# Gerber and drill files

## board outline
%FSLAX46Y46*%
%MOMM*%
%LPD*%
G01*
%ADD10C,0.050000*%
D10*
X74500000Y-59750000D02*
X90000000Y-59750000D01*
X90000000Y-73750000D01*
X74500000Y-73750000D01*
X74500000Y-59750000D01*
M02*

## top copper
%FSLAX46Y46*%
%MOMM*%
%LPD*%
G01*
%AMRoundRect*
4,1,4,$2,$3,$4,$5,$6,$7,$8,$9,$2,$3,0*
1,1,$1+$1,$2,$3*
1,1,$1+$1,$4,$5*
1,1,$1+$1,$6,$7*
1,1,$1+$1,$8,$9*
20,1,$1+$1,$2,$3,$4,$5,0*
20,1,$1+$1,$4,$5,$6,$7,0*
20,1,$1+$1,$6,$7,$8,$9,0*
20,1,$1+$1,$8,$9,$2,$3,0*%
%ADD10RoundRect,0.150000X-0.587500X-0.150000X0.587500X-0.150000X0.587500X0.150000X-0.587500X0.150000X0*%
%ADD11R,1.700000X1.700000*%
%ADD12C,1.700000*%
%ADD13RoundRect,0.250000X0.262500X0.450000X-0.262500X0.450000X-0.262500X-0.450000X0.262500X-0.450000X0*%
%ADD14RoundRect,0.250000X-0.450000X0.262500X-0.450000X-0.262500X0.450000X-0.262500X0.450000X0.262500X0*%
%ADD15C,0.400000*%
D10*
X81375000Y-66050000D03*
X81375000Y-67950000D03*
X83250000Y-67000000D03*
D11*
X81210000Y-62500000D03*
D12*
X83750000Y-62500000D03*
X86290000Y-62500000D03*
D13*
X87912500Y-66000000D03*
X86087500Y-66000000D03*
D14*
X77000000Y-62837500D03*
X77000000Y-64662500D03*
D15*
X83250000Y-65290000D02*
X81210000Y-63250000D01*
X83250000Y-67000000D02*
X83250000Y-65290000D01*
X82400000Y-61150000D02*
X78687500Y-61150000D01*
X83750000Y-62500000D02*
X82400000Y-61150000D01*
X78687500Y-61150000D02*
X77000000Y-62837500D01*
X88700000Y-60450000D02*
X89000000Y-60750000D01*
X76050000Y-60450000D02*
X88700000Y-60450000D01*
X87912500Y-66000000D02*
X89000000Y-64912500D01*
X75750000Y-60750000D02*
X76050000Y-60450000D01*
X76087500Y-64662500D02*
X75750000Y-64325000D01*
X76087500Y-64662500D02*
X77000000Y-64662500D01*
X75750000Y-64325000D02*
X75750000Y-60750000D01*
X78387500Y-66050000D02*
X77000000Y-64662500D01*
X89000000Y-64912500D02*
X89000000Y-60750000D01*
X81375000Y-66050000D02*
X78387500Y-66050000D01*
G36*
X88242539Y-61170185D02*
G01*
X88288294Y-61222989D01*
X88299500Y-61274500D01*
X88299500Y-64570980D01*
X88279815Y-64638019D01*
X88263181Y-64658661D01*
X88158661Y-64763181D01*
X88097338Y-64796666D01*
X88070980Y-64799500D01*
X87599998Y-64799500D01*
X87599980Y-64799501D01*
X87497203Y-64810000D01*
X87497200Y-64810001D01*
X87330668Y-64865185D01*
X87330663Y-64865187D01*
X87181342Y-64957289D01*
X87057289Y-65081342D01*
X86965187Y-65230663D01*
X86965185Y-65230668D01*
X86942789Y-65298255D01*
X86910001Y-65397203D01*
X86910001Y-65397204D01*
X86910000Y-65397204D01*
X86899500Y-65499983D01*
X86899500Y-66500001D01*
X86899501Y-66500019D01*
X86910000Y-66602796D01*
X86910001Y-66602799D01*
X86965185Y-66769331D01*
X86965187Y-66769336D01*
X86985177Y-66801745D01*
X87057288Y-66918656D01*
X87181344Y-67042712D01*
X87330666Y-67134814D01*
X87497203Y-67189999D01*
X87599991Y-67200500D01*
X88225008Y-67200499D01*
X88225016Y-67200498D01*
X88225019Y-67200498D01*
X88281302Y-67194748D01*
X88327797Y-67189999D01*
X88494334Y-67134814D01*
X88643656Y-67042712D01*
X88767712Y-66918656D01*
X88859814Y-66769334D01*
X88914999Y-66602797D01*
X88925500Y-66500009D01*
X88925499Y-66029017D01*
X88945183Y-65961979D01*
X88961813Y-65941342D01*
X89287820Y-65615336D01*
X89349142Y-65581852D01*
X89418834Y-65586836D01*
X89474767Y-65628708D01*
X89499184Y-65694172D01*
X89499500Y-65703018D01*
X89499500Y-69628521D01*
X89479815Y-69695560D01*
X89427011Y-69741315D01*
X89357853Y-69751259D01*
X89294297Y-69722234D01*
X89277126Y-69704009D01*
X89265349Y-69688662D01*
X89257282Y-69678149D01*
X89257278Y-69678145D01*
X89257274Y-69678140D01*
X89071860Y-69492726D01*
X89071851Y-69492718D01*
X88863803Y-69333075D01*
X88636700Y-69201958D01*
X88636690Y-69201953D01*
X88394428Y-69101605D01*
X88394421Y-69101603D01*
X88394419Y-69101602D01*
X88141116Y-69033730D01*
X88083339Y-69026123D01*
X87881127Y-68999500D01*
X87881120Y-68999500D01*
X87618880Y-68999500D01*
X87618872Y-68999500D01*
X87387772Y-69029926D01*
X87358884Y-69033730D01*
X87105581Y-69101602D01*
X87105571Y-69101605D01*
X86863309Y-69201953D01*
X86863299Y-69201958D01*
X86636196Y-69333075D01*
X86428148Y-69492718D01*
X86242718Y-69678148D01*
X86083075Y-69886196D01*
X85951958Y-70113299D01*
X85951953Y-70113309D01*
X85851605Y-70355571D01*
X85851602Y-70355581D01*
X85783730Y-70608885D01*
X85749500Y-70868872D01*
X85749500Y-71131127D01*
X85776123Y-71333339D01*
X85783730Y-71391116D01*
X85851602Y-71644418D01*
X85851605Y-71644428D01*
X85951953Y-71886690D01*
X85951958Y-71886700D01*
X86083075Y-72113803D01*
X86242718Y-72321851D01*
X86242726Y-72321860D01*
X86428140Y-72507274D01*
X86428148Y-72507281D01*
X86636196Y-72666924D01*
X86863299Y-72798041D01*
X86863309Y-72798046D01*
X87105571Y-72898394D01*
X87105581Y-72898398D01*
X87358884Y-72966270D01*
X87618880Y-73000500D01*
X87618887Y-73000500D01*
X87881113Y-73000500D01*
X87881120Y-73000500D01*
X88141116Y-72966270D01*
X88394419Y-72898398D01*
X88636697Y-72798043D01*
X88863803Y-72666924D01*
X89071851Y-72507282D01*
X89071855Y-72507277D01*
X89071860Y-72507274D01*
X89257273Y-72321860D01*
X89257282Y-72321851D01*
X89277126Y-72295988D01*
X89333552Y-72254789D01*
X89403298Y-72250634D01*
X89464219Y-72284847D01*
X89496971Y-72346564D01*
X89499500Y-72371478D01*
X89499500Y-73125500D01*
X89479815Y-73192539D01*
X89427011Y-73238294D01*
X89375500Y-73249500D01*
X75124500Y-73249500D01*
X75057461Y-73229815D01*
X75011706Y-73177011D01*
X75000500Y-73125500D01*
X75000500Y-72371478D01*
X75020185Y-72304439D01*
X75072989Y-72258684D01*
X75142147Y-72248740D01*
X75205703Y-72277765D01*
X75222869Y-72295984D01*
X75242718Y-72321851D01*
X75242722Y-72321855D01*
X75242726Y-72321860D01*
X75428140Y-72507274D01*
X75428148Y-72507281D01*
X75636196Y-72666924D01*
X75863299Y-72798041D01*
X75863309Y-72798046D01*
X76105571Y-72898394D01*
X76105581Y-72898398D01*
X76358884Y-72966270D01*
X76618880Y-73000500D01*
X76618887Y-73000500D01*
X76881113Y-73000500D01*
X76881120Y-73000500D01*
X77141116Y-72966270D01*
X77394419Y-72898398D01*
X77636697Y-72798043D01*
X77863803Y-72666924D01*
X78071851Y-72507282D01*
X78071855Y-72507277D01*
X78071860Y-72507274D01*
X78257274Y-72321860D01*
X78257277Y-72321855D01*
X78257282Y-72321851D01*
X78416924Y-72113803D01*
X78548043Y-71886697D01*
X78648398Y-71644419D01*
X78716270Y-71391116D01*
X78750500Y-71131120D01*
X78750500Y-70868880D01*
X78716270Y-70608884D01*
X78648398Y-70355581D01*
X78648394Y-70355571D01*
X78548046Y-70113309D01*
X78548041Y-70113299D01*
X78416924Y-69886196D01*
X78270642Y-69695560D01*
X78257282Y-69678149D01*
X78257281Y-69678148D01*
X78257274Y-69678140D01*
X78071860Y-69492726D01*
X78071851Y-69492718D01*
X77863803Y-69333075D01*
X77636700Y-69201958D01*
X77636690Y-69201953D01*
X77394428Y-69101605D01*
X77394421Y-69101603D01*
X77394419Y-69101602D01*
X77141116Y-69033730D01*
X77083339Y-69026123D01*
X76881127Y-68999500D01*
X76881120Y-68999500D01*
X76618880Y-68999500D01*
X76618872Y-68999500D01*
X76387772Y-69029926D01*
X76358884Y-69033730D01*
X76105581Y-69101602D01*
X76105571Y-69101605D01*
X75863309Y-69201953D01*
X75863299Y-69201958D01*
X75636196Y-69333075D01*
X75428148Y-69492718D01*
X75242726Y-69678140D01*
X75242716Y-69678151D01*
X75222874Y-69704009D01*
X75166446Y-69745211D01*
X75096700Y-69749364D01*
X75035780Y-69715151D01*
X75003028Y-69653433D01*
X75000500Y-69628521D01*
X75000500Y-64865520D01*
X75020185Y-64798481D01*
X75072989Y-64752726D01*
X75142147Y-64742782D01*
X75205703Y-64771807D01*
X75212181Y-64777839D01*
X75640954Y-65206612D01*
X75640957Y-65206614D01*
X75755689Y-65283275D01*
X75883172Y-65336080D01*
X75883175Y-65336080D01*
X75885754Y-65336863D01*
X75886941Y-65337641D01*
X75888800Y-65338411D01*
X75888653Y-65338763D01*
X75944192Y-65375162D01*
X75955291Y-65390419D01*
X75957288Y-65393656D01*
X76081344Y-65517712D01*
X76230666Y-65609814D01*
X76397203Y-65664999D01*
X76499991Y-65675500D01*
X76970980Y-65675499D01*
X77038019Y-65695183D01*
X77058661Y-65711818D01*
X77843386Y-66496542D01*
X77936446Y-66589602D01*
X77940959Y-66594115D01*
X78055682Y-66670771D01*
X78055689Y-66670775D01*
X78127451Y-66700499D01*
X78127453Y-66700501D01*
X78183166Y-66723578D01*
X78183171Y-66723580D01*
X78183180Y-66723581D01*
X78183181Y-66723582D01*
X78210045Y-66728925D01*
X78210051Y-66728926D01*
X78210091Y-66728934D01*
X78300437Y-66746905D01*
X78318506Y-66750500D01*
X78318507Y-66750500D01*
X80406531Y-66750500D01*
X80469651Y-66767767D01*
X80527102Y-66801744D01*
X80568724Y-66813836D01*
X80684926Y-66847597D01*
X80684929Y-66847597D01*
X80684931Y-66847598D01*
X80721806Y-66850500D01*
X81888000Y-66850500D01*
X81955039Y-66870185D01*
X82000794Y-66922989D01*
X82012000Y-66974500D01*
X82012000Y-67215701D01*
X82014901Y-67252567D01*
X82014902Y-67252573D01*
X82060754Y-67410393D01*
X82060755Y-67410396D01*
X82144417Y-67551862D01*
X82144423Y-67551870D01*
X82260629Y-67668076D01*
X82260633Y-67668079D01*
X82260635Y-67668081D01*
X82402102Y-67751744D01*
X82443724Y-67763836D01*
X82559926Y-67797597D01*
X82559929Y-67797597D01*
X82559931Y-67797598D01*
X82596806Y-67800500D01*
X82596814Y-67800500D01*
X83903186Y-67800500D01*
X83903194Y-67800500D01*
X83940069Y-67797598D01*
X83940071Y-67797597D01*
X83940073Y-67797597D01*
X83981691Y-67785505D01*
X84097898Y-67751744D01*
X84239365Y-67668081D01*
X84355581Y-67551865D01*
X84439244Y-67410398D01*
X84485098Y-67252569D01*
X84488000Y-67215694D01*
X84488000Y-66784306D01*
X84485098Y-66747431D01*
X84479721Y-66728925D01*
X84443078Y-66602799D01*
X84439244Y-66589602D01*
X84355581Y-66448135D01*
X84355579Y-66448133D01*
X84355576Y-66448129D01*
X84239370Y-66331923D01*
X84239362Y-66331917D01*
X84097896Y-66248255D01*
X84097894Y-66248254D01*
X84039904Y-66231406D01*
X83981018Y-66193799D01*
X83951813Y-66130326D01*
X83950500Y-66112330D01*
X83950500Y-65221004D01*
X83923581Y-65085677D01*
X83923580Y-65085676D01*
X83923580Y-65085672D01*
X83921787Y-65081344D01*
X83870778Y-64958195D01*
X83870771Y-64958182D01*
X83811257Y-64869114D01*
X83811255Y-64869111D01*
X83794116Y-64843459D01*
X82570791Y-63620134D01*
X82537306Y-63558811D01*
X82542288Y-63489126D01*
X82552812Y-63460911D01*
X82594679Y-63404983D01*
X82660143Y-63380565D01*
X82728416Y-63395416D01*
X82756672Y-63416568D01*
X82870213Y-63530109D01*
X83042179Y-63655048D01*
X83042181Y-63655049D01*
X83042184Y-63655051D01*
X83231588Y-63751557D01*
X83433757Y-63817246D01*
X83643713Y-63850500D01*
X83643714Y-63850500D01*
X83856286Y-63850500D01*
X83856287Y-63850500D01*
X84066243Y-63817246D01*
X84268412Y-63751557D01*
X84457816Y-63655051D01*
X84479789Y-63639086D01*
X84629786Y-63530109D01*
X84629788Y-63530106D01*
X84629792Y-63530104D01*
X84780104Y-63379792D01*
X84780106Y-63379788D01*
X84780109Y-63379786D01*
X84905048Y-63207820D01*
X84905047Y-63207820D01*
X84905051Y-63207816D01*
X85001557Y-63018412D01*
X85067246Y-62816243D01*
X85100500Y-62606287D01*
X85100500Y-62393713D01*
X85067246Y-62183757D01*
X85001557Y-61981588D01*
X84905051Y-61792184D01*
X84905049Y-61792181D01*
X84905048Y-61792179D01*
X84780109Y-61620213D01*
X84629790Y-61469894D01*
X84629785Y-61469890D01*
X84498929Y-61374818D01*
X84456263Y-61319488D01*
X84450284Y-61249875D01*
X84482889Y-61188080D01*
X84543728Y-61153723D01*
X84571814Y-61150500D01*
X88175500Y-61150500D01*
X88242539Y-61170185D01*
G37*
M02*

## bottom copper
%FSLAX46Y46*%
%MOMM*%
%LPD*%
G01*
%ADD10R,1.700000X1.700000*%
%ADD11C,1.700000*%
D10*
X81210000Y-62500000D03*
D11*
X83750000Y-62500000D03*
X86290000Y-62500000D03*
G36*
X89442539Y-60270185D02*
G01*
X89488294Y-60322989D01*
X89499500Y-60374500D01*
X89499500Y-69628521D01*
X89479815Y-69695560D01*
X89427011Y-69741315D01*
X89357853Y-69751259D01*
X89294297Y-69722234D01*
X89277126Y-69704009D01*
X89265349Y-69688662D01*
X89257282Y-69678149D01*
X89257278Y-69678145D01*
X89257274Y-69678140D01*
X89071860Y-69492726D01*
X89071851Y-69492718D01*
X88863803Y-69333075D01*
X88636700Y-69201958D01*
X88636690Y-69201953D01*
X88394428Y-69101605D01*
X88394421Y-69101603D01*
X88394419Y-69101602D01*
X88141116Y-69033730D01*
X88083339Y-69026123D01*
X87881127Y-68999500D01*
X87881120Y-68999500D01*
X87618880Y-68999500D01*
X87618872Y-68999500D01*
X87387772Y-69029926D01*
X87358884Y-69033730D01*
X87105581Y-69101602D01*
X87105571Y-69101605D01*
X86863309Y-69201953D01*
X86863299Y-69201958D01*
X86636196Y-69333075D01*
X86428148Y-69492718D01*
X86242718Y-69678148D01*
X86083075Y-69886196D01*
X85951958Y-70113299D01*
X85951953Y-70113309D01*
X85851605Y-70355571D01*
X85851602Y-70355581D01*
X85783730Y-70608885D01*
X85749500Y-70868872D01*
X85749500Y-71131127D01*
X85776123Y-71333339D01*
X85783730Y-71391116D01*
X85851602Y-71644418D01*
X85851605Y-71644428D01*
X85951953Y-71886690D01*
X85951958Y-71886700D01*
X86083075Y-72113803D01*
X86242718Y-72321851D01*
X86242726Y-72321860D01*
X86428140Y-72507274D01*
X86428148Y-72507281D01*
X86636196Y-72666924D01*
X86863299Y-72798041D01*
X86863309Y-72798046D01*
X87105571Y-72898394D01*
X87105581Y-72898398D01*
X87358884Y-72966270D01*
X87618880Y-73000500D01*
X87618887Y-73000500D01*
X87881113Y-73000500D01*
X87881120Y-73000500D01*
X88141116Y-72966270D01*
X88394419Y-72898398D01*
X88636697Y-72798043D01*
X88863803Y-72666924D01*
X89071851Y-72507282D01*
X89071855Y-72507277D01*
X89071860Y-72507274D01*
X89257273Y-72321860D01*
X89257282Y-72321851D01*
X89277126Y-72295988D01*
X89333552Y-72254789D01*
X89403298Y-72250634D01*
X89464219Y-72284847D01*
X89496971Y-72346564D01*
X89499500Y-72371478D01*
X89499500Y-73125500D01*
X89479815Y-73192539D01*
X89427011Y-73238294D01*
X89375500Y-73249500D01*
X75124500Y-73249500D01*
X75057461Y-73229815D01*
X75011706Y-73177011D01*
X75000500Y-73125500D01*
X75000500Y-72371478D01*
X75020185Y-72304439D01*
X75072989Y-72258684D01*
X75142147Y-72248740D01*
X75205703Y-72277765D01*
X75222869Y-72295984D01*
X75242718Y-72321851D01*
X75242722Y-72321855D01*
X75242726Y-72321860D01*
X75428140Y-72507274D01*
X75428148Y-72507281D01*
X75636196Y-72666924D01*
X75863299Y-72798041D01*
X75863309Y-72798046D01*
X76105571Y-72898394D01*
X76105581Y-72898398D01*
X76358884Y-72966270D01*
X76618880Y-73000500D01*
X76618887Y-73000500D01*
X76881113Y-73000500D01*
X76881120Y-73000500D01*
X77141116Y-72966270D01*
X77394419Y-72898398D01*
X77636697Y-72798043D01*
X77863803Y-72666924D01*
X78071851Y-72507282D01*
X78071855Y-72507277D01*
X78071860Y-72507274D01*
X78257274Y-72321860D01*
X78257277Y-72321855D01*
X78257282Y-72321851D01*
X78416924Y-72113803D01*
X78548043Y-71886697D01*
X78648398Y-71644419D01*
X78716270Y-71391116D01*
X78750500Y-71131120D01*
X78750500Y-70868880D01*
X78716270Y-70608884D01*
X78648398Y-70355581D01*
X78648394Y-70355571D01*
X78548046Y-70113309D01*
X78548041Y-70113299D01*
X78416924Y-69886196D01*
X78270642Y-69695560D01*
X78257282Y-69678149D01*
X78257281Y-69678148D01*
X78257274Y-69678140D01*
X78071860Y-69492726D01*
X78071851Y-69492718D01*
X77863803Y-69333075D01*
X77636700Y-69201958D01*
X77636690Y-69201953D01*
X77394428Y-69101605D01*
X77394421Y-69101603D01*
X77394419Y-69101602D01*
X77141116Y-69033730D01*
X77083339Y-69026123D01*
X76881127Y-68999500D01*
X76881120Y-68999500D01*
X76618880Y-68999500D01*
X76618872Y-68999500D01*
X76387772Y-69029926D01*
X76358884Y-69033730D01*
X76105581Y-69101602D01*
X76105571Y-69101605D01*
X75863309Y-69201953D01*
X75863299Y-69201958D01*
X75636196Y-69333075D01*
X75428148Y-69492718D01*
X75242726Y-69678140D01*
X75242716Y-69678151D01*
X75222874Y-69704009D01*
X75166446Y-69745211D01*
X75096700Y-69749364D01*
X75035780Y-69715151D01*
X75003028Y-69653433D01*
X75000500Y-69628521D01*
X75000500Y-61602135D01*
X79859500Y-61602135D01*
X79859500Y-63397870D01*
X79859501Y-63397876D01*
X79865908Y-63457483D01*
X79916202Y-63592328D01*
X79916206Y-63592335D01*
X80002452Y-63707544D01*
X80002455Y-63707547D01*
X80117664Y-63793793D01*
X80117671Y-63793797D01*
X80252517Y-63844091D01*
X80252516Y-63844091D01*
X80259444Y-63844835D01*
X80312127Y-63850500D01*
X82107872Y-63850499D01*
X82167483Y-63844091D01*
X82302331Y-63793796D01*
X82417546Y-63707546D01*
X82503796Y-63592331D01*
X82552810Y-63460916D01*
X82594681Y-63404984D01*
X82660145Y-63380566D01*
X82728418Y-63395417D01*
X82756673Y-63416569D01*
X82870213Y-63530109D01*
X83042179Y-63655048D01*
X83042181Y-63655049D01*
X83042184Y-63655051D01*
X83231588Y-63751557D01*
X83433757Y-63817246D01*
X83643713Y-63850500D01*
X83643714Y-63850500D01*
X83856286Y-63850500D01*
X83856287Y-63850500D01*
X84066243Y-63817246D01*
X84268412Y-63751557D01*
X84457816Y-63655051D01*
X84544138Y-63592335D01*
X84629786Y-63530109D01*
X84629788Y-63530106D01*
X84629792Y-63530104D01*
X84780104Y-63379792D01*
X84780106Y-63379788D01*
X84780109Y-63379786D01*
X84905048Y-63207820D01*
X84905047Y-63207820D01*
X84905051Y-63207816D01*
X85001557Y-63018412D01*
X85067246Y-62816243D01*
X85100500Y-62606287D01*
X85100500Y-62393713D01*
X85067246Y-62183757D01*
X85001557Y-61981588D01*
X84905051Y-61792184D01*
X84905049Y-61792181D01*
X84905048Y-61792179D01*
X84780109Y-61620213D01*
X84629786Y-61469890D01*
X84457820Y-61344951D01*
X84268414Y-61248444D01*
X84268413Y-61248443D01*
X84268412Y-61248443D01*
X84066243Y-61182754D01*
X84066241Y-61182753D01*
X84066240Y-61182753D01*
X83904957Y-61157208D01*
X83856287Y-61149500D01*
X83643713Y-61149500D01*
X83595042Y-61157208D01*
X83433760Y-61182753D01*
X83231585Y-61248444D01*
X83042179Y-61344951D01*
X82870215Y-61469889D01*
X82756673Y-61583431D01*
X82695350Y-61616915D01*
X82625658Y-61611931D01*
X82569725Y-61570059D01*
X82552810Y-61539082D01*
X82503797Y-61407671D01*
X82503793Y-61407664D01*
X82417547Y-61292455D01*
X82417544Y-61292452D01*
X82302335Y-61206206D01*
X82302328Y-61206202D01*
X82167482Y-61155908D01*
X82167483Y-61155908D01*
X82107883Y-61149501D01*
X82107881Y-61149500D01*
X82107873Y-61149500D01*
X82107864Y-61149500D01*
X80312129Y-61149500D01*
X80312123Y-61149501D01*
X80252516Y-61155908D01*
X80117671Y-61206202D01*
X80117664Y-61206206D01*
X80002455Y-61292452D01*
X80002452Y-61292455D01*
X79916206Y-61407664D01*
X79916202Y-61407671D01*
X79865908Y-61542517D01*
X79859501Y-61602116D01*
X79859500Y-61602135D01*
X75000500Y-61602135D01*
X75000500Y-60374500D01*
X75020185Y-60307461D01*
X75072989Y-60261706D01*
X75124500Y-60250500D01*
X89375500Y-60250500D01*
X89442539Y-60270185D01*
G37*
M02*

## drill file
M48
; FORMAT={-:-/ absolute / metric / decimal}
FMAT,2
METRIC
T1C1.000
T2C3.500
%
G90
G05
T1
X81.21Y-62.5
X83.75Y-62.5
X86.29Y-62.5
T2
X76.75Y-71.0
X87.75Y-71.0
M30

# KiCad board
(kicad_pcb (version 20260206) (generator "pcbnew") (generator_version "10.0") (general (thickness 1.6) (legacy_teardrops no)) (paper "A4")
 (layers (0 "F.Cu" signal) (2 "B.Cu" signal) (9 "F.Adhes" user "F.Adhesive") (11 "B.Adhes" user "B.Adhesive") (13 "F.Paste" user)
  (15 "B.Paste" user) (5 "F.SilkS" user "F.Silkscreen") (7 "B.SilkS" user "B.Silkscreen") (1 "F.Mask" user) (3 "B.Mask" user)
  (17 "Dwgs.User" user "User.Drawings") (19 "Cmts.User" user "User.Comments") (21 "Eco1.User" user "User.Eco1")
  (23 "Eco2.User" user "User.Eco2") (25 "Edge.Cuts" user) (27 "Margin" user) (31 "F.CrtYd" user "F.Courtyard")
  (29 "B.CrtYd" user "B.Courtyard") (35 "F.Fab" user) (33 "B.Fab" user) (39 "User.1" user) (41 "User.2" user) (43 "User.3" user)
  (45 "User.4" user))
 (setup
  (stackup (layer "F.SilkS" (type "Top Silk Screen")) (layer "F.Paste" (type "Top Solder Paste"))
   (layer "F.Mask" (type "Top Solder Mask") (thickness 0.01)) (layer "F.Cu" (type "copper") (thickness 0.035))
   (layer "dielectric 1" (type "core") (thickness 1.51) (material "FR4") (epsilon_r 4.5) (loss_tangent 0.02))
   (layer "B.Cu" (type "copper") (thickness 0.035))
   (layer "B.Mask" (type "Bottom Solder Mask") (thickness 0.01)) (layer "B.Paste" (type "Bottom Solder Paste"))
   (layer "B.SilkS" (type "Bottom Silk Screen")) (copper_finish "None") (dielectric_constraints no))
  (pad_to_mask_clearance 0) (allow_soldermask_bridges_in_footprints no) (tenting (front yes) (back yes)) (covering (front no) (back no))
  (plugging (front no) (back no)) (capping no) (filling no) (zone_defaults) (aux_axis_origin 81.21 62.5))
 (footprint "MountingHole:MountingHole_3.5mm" (layer "F.Cu") (at 87.75 71)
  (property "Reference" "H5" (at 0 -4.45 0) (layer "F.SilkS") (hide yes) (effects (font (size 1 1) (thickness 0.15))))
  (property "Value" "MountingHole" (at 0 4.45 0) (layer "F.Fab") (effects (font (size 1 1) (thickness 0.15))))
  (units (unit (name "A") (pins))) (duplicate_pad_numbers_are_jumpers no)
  (pad "" np_thru_hole circle (at 0 0) (size 3.5 3.5) (drill 3.5) (layers "*.Cu" "*.Mask")))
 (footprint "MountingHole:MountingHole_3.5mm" (layer "F.Cu") (at 76.75 71)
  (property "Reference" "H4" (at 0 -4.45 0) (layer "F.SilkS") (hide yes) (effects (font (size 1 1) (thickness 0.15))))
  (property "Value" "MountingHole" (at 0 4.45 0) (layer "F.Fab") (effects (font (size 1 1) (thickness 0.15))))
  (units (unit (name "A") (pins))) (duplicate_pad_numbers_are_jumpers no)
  (pad "" np_thru_hole circle (at 0 0) (size 3.5 3.5) (drill 3.5) (layers "*.Cu" "*.Mask")))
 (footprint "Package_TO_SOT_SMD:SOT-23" (layer "F.Cu") (at 82.3125 67)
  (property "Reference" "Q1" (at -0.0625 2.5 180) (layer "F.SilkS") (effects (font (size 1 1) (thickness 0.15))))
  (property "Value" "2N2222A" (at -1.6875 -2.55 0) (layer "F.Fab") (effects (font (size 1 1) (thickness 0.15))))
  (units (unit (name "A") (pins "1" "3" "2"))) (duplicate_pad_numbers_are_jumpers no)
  (pad "1" smd roundrect (at -0.9375 -0.95) (size 1.475 0.6) (layers "F.Cu" "F.Mask" "F.Paste") (roundrect_rratio 0.25) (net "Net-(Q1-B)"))
  (pad "2" smd roundrect (at -0.9375 0.95) (size 1.475 0.6) (layers "F.Cu" "F.Mask" "F.Paste") (roundrect_rratio 0.25) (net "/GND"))
  (pad "3" smd roundrect (at 0.9375 0) (size 1.475 0.6) (layers "F.Cu" "F.Mask" "F.Paste") (roundrect_rratio 0.25) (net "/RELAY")))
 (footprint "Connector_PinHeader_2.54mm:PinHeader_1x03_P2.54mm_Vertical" (layer "F.Cu") (at 81.21 62.5 90)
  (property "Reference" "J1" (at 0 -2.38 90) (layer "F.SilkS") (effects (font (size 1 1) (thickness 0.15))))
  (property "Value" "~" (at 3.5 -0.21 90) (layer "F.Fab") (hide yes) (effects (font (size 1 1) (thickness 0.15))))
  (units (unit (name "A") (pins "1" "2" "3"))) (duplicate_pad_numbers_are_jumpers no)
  (pad "1" thru_hole rect (at 0 0 90) (size 1.7 1.7) (drill 1) (layers "*.Cu" "*.Mask") (remove_unused_layers no) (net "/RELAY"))
  (pad "2" thru_hole circle (at 0 2.54 90) (size 1.7 1.7) (drill 1) (layers "*.Cu" "*.Mask") (remove_unused_layers no) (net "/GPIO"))
  (pad "3" thru_hole circle (at 0 5.08 90) (size 1.7 1.7) (drill 1) (layers "*.Cu" "*.Mask") (remove_unused_layers no) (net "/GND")))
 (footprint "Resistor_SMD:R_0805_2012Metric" (layer "F.Cu") (at 87 66 180)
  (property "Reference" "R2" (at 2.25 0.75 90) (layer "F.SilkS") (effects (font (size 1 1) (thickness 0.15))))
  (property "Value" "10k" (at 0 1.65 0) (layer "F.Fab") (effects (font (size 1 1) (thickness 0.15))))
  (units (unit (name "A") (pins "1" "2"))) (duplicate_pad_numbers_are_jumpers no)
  (pad "1" smd roundrect (at -0.9125 0 180) (size 1.025 1.4) (layers "F.Cu" "F.Mask" "F.Paste") (roundrect_rratio 0.243902)
   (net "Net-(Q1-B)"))
  (pad "2" smd roundrect (at 0.9125 0 180) (size 1.025 1.4) (layers "F.Cu" "F.Mask" "F.Paste") (roundrect_rratio 0.243902) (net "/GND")))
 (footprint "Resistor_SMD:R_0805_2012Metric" (layer "F.Cu") (at 77 63.75 -90)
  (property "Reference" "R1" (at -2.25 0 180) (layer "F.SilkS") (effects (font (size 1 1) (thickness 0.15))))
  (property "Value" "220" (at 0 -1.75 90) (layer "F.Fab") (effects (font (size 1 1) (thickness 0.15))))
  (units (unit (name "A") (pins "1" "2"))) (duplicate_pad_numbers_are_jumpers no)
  (pad "1" smd roundrect (at -0.9125 0 270) (size 1.025 1.4) (layers "F.Cu" "F.Mask" "F.Paste") (roundrect_rratio 0.243902) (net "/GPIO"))
  (pad "2" smd roundrect (at 0.9125 0 270) (size 1.025 1.4) (layers "F.Cu" "F.Mask" "F.Paste") (roundrect_rratio 0.243902)
   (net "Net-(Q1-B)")))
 (gr_rect (start 74.5 59.75) (end 90 73.75) (stroke (width 0.05) (type default)) (fill no) (layer "Edge.Cuts"))
 (segment (start 83.25 65.29) (end 81.21 63.25) (width 0.4) (layer "F.Cu") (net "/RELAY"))
 (segment (start 83.25 67) (end 83.25 65.29) (width 0.4) (layer "F.Cu") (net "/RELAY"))
 (segment (start 82.4 61.15) (end 78.6875 61.15) (width 0.4) (layer "F.Cu") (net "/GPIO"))
 (segment (start 83.75 62.5) (end 82.4 61.15) (width 0.4) (layer "F.Cu") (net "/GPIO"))
 (segment (start 78.6875 61.15) (end 77 62.8375) (width 0.4) (layer "F.Cu") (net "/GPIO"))
 (segment (start 88.7 60.45) (end 89 60.75) (width 0.4) (layer "F.Cu") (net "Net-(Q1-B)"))
 (segment (start 76.05 60.45) (end 88.7 60.45) (width 0.4) (layer "F.Cu") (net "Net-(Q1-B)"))
 (segment (start 87.9125 66) (end 89 64.9125) (width 0.4) (layer "F.Cu") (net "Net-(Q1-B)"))
 (segment (start 75.75 60.75) (end 76.05 60.45) (width 0.4) (layer "F.Cu") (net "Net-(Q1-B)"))
 (segment (start 76.0875 64.6625) (end 75.75 64.325) (width 0.4) (layer "F.Cu") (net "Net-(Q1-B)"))
 (segment (start 76.0875 64.6625) (end 77 64.6625) (width 0.4) (layer "F.Cu") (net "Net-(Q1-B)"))
 (segment (start 75.75 64.325) (end 75.75 60.75) (width 0.4) (layer "F.Cu") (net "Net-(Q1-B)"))
 (segment (start 78.3875 66.05) (end 77 64.6625) (width 0.4) (layer "F.Cu") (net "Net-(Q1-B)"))
 (segment (start 89 64.9125) (end 89 60.75) (width 0.4) (layer "F.Cu") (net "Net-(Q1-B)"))
 (segment (start 81.375 66.05) (end 78.3875 66.05) (width 0.4) (layer "F.Cu") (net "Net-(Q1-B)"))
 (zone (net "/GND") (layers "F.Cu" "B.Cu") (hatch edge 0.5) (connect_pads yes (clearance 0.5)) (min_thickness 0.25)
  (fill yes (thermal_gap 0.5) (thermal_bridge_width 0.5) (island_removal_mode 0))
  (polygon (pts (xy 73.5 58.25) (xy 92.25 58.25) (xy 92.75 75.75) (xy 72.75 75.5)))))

